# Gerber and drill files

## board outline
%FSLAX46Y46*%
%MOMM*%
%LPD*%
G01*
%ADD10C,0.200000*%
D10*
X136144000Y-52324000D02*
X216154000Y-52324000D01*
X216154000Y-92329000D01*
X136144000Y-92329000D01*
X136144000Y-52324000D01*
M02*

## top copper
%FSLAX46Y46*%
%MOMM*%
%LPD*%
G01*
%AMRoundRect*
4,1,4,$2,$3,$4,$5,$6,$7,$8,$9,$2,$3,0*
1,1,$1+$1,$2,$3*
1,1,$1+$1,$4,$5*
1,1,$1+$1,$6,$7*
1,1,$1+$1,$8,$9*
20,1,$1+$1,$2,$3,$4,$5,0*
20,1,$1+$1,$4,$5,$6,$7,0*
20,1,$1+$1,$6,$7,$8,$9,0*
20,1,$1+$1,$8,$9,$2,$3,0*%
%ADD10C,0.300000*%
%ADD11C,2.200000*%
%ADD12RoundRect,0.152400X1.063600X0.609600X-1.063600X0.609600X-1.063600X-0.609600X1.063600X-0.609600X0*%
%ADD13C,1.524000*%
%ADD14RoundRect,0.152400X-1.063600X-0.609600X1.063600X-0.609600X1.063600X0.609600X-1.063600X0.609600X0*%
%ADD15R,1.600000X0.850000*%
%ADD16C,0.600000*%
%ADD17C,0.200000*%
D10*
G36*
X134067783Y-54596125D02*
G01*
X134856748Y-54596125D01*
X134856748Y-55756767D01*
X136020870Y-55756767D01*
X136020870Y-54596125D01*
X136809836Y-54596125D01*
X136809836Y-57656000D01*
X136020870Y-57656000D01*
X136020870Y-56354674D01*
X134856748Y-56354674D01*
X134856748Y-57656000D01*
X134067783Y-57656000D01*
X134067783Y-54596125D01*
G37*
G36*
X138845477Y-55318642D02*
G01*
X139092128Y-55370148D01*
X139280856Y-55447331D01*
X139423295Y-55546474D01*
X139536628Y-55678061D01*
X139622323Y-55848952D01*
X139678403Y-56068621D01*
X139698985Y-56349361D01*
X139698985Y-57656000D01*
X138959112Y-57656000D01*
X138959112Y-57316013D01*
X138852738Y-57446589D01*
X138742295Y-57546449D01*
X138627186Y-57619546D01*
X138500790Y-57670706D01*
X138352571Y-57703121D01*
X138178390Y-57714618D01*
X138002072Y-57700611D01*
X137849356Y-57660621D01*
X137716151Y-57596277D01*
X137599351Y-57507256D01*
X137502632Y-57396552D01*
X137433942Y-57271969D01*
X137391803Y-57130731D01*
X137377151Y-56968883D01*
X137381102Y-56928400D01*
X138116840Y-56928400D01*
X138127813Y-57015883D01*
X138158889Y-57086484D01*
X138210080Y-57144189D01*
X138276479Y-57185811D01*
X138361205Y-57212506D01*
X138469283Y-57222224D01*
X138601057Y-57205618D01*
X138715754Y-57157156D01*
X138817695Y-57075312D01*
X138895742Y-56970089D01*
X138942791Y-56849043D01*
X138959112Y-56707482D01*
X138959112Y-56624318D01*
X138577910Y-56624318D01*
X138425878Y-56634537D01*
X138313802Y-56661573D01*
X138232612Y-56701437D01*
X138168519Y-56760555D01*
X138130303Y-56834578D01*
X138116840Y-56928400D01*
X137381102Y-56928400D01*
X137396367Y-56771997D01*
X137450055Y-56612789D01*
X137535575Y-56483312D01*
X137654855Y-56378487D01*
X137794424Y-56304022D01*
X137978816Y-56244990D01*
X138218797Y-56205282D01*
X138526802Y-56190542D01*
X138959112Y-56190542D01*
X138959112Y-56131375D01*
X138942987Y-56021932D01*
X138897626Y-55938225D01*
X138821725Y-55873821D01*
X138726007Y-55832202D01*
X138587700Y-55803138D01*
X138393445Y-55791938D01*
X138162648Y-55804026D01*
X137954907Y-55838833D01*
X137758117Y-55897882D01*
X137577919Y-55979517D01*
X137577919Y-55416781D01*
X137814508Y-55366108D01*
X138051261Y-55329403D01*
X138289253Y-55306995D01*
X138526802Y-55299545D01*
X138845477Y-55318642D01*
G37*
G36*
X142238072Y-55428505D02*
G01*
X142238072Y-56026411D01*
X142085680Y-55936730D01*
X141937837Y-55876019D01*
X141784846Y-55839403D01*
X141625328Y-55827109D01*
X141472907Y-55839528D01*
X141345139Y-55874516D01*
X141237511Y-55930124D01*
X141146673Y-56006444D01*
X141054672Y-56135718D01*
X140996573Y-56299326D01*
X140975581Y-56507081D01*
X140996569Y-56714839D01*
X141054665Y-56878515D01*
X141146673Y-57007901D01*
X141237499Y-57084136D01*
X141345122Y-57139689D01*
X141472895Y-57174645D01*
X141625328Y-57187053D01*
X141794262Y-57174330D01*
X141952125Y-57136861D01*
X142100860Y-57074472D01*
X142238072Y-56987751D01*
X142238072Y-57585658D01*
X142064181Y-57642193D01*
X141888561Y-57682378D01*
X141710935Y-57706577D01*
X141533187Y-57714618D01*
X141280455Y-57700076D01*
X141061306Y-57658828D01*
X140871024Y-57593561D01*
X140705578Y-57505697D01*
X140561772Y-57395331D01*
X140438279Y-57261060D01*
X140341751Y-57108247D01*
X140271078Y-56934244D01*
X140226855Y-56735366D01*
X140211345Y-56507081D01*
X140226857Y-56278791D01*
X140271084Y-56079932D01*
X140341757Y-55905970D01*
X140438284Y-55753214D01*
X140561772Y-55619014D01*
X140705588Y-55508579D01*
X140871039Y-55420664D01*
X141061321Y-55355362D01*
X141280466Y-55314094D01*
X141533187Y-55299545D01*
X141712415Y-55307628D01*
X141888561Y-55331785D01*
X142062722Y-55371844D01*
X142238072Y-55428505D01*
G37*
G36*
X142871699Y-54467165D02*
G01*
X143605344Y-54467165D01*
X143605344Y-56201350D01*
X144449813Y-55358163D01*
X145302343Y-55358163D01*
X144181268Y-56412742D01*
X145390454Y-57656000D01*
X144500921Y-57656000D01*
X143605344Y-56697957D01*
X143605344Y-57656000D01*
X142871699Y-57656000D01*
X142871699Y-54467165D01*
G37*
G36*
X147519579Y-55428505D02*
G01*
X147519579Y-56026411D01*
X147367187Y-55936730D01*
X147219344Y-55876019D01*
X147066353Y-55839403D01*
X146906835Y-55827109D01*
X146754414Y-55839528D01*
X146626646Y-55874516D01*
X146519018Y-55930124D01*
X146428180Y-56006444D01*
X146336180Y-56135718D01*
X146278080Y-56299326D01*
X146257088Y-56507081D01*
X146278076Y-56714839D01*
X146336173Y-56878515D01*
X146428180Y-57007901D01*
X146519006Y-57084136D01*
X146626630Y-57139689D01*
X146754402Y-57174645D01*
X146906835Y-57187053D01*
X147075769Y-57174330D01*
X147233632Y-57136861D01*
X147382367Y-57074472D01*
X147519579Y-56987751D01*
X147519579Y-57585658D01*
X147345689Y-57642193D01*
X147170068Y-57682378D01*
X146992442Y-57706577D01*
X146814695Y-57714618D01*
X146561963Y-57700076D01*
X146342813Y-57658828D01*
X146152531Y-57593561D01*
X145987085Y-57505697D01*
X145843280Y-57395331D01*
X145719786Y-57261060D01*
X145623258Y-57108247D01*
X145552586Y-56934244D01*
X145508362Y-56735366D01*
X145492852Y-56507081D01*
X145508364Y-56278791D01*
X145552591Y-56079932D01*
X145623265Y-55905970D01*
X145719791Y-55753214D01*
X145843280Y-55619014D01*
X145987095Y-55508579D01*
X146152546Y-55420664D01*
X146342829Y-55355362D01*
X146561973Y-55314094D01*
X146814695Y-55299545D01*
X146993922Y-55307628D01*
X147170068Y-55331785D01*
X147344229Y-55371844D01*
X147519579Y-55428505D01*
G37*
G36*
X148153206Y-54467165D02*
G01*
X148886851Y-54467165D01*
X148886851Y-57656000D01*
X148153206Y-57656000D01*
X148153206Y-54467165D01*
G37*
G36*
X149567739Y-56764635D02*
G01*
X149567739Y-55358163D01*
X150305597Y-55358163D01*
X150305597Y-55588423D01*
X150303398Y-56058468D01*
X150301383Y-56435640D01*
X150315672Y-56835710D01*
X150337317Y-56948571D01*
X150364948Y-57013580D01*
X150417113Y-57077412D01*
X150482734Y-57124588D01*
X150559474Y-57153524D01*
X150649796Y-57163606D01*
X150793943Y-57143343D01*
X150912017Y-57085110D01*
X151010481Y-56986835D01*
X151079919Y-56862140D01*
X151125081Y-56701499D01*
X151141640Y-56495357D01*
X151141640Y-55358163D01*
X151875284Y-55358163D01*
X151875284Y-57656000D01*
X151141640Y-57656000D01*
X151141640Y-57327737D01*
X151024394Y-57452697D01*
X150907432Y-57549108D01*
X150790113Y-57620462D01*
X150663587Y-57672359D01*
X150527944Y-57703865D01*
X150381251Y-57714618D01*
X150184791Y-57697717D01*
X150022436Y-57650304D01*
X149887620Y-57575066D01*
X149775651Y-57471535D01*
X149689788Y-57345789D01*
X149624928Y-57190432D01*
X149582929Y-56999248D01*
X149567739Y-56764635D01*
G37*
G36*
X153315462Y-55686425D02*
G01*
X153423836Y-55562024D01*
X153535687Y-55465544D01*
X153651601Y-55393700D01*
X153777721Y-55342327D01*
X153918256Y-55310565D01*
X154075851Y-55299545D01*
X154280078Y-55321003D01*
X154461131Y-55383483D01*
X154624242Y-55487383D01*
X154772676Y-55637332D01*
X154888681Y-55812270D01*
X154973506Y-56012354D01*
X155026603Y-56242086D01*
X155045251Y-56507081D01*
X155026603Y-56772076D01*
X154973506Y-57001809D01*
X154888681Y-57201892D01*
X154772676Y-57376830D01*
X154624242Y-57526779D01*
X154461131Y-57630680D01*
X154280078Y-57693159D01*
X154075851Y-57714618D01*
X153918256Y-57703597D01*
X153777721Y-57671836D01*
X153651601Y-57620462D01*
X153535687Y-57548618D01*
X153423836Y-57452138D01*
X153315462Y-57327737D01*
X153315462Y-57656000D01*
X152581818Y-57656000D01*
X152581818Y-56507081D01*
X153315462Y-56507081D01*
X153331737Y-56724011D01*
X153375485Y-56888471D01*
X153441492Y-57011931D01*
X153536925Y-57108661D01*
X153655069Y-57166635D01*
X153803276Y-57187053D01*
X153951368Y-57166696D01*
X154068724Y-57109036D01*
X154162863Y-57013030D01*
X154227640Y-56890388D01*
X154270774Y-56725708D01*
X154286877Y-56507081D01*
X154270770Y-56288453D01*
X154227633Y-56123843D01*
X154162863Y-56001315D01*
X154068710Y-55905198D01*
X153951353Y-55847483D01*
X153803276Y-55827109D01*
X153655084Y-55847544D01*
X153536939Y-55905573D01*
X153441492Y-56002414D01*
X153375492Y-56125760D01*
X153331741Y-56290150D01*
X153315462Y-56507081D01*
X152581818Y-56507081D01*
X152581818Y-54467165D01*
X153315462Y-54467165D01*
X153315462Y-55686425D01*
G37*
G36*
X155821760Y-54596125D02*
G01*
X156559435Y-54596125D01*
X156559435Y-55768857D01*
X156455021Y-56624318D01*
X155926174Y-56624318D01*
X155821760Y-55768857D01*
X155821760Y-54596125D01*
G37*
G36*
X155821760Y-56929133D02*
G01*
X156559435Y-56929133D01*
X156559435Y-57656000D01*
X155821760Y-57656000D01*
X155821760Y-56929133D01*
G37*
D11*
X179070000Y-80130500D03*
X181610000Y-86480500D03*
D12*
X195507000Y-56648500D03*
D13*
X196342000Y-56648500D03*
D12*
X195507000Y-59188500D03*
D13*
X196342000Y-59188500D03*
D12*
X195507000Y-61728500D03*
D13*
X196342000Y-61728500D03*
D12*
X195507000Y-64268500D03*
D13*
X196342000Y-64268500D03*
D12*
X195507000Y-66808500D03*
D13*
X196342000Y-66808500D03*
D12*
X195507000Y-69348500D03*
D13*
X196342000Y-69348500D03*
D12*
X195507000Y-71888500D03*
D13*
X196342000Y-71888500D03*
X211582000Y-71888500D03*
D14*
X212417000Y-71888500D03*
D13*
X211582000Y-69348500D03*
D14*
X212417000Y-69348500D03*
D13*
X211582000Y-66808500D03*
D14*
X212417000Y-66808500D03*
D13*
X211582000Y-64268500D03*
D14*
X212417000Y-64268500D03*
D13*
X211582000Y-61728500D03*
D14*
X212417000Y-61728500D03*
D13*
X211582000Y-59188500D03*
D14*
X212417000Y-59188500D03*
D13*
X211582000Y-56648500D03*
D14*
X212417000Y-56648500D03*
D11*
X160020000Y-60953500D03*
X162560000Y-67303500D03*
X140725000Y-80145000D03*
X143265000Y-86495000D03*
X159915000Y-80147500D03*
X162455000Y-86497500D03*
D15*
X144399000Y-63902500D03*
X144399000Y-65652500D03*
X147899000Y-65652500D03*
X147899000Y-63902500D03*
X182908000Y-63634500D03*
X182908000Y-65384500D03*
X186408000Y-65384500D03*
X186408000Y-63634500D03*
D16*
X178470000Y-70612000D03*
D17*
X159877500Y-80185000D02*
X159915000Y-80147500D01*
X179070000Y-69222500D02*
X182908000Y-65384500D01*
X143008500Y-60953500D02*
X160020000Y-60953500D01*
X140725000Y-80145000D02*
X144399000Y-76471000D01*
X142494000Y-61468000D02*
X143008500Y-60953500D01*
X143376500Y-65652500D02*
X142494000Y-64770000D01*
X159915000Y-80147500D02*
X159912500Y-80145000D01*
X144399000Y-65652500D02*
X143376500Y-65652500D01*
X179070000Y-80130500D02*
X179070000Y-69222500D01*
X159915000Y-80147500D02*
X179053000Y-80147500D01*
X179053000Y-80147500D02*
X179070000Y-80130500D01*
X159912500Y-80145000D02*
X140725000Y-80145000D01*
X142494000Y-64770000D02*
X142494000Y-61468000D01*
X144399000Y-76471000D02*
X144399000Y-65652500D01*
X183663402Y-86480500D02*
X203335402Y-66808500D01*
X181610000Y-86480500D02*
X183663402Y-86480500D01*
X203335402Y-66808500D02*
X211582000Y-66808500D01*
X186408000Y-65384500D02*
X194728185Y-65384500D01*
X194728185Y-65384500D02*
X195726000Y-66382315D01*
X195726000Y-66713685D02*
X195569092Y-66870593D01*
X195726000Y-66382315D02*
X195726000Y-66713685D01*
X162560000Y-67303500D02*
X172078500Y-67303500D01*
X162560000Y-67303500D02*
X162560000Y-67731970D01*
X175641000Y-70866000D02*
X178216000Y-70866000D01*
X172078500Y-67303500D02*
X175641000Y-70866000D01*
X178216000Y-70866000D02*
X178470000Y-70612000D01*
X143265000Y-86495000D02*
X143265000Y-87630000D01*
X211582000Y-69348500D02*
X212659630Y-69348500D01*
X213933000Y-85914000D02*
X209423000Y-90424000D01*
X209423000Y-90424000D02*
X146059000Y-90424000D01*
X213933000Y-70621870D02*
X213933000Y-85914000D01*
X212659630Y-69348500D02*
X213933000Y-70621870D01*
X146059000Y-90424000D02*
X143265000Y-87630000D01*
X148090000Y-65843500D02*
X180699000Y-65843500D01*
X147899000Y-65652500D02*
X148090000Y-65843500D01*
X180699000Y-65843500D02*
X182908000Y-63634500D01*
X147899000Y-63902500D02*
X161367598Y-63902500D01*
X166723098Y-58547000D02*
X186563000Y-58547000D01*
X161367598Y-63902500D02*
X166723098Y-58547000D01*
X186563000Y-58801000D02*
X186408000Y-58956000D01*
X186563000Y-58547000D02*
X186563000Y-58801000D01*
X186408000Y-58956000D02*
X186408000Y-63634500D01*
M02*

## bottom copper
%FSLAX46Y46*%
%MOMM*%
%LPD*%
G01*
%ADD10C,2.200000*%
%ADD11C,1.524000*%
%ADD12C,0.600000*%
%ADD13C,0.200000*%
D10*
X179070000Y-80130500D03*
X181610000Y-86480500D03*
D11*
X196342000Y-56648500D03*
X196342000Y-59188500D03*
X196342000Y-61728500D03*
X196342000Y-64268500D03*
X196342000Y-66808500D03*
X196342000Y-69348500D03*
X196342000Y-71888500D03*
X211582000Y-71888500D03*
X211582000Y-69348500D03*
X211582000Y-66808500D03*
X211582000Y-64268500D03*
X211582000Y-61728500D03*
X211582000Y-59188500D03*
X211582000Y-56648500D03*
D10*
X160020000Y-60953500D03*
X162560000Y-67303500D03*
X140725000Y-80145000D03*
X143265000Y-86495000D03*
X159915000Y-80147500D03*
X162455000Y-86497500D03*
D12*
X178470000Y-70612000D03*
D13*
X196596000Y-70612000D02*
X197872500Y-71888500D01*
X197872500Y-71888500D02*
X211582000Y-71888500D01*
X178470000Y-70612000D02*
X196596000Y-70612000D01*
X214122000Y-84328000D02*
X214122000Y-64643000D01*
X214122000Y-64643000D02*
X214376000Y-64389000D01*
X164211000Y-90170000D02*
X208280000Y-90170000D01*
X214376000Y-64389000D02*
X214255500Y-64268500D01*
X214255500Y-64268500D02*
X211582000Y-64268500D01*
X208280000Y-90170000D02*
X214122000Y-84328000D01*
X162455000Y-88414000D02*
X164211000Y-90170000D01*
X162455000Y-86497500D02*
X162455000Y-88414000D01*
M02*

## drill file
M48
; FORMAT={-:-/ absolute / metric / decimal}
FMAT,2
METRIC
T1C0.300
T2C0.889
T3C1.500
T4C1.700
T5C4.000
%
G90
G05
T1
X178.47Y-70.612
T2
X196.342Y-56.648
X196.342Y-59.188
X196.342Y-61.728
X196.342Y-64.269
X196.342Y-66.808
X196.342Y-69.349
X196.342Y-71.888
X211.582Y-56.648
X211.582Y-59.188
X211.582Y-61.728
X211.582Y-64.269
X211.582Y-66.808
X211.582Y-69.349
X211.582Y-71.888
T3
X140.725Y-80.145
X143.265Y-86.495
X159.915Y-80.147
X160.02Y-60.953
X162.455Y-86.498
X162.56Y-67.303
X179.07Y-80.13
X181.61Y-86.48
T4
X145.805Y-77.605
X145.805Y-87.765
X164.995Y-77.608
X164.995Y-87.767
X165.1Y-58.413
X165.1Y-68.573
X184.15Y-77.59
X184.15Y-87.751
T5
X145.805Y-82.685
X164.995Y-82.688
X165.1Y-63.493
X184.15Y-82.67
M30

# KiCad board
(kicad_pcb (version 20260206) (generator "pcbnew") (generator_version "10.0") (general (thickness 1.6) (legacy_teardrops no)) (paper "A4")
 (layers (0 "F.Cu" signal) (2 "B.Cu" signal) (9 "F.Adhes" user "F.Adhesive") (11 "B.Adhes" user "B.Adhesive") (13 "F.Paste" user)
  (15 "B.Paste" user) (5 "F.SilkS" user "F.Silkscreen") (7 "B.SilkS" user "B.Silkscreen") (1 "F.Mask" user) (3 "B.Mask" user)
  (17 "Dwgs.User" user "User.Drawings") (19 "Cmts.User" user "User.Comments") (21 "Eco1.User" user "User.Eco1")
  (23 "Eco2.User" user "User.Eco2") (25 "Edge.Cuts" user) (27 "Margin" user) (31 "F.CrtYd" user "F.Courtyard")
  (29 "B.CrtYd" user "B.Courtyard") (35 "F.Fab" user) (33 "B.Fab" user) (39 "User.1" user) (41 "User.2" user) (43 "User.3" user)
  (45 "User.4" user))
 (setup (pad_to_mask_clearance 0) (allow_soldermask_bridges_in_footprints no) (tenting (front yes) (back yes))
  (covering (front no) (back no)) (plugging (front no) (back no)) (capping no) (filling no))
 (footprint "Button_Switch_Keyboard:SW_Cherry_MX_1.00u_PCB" (layer "F.Cu") (at 179.07 80.1305 90)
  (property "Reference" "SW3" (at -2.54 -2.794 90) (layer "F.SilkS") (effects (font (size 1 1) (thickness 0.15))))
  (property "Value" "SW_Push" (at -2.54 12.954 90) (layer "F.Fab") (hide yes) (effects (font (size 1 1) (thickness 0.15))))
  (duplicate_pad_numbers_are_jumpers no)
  (pad "" np_thru_hole circle (at -7.62 5.08 90) (size 1.7 1.7) (drill 1.7) (layers "*.Cu" "*.Mask"))
  (pad "" np_thru_hole circle (at -2.54 5.08 90) (size 4 4) (drill 4) (layers "*.Cu" "*.Mask"))
  (pad "" np_thru_hole circle (at 2.54 5.08 90) (size 1.7 1.7) (drill 1.7) (layers "*.Cu" "*.Mask"))
  (pad "1" thru_hole circle (at 0 0 90) (size 2.2 2.2) (drill 1.5) (layers "*.Cu" "*.Mask") (remove_unused_layers no) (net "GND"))
  (pad "2" thru_hole circle (at -6.35 2.54 90) (size 2.2 2.2) (drill 1.5) (layers "*.Cu" "*.Mask") (remove_unused_layers no)
   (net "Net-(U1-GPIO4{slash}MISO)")))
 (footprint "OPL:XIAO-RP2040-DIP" (layer "F.Cu") (at 203.962 64.2685)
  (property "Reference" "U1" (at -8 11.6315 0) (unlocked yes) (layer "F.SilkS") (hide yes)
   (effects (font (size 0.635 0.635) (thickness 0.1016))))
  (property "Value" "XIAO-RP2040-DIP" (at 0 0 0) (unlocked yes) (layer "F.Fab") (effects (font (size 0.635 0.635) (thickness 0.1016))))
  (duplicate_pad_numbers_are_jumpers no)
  (pad "1" smd roundrect (at -8.455 -7.62 180) (size 2.432 1.524) (layers "F.Cu" "F.Mask") (roundrect_rratio 0.1)
   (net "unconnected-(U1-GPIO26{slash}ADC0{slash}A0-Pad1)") (thermal_bridge_angle 45))
  (pad "1" thru_hole circle (at -7.62 -7.62 180) (size 1.524 1.524) (drill 0.889) (layers "*.Cu" "*.Mask") (remove_unused_layers no)
   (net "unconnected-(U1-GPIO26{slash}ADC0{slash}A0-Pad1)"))
  (pad "2" smd roundrect (at -8.455 -5.08 180) (size 2.432 1.524) (layers "F.Cu" "F.Mask") (roundrect_rratio 0.1)
   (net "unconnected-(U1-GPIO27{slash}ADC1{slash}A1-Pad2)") (thermal_bridge_angle 45))
  (pad "2" thru_hole circle (at -7.62 -5.08 180) (size 1.524 1.524) (drill 0.889) (layers "*.Cu" "*.Mask") (remove_unused_layers no)
   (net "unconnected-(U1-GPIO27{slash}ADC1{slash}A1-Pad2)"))
  (pad "3" smd roundrect (at -8.455 -2.54 180) (size 2.432 1.524) (layers "F.Cu" "F.Mask") (roundrect_rratio 0.1)
   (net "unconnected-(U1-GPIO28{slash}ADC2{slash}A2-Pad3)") (thermal_bridge_angle 45))
  (pad "3" thru_hole circle (at -7.62 -2.54 180) (size 1.524 1.524) (drill 0.889) (layers "*.Cu" "*.Mask") (remove_unused_layers no)
   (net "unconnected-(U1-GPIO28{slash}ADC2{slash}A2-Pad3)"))
  (pad "4" smd roundrect (at -8.455 0 180) (size 2.432 1.524) (layers "F.Cu" "F.Mask") (roundrect_rratio 0.1)
   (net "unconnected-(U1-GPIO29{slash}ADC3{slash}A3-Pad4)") (thermal_bridge_angle 45))
  (pad "4" thru_hole circle (at -7.62 0 180) (size 1.524 1.524) (drill 0.889) (layers "*.Cu" "*.Mask") (remove_unused_layers no)
   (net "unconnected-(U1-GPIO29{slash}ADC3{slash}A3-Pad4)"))
  (pad "5" smd roundrect (at -8.455 2.54 180) (size 2.432 1.524) (layers "F.Cu" "F.Mask") (roundrect_rratio 0.1) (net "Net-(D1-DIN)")
   (thermal_bridge_angle 45))
  (pad "5" thru_hole circle (at -7.62 2.54 180) (size 1.524 1.524) (drill 0.889) (layers "*.Cu" "*.Mask") (remove_unused_layers no)
   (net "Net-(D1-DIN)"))
  (pad "6" smd roundrect (at -8.455 5.08 180) (size 2.432 1.524) (layers "F.Cu" "F.Mask") (roundrect_rratio 0.1)
   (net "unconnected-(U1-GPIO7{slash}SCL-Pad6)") (thermal_bridge_angle 45))
  (pad "6" thru_hole circle (at -7.62 5.08 180) (size 1.524 1.524) (drill 0.889) (layers "*.Cu" "*.Mask") (remove_unused_layers no)
   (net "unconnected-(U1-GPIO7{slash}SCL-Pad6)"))
  (pad "7" smd roundrect (at -8.455 7.62 180) (size 2.432 1.524) (layers "F.Cu" "F.Mask") (roundrect_rratio 0.1)
   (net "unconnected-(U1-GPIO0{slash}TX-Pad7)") (thermal_bridge_angle 45))
  (pad "7" thru_hole circle (at -7.62 7.62 180) (size 1.524 1.524) (drill 0.889) (layers "*.Cu" "*.Mask") (remove_unused_layers no)
   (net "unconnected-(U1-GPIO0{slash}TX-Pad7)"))
  (pad "8" thru_hole circle (at 7.62 7.62) (size 1.524 1.524) (drill 0.889) (layers "*.Cu" "*.Mask") (remove_unused_layers no)
   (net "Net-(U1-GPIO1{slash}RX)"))
  (pad "8" smd roundrect (at 8.455 7.62) (size 2.432 1.524) (layers "F.Cu" "F.Mask") (roundrect_rratio 0.1) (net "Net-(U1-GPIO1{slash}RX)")
   (thermal_bridge_angle 45))
  (pad "9" thru_hole circle (at 7.62 5.08) (size 1.524 1.524) (drill 0.889) (layers "*.Cu" "*.Mask") (remove_unused_layers no)
   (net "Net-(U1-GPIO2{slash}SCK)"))
  (pad "9" smd roundrect (at 8.455 5.08) (size 2.432 1.524) (layers "F.Cu" "F.Mask") (roundrect_rratio 0.1) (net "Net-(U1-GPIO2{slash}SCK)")
   (thermal_bridge_angle 45))
  (pad "10" thru_hole circle (at 7.62 2.54) (size 1.524 1.524) (drill 0.889) (layers "*.Cu" "*.Mask") (remove_unused_layers no)
   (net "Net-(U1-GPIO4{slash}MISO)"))
  (pad "10" smd roundrect (at 8.455 2.54) (size 2.432 1.524) (layers "F.Cu" "F.Mask") (roundrect_rratio 0.1)
   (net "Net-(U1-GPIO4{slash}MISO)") (thermal_bridge_angle 45))
  (pad "11" thru_hole circle (at 7.62 0) (size 1.524 1.524) (drill 0.889) (layers "*.Cu" "*.Mask") (remove_unused_layers no)
   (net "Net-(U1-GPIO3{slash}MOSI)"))
  (pad "11" smd roundrect (at 8.455 0) (size 2.432 1.524) (layers "F.Cu" "F.Mask") (roundrect_rratio 0.1) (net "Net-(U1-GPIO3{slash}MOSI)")
   (thermal_bridge_angle 45))
  (pad "12" thru_hole circle (at 7.62 -2.54) (size 1.524 1.524) (drill 0.889) (layers "*.Cu" "*.Mask") (remove_unused_layers no)
   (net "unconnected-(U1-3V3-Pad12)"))
  (pad "12" smd roundrect (at 8.455 -2.54) (size 2.432 1.524) (layers "F.Cu" "F.Mask") (roundrect_rratio 0.1)
   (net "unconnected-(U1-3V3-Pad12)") (thermal_bridge_angle 45))
  (pad "13" thru_hole circle (at 7.62 -5.08) (size 1.524 1.524) (drill 0.889) (layers "*.Cu" "*.Mask") (remove_unused_layers no)
   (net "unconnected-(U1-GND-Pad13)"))
  (pad "13" smd roundrect (at 8.455 -5.08) (size 2.432 1.524) (layers "F.Cu" "F.Mask") (roundrect_rratio 0.1)
   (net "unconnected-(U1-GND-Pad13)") (thermal_bridge_angle 45))
  (pad "14" thru_hole circle (at 7.62 -7.62) (size 1.524 1.524) (drill 0.889) (layers "*.Cu" "*.Mask") (remove_unused_layers no)
   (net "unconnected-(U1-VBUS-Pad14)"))
  (pad "14" smd roundrect (at 8.455 -7.62) (size 2.432 1.524) (layers "F.Cu" "F.Mask") (roundrect_rratio 0.1)
   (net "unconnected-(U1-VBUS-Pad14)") (thermal_bridge_angle 45)))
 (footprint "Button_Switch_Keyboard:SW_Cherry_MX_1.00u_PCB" (layer "F.Cu") (at 160.02 60.9535 90)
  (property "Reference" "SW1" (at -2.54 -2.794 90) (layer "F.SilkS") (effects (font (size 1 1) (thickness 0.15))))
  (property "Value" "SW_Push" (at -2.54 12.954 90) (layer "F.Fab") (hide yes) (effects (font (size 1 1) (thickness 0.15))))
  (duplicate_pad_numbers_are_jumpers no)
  (pad "" np_thru_hole circle (at -7.62 5.08 90) (size 1.7 1.7) (drill 1.7) (layers "*.Cu" "*.Mask"))
  (pad "" np_thru_hole circle (at -2.54 5.08 90) (size 4 4) (drill 4) (layers "*.Cu" "*.Mask"))
  (pad "" np_thru_hole circle (at 2.54 5.08 90) (size 1.7 1.7) (drill 1.7) (layers "*.Cu" "*.Mask"))
  (pad "1" thru_hole circle (at 0 0 90) (size 2.2 2.2) (drill 1.5) (layers "*.Cu" "*.Mask") (remove_unused_layers no) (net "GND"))
  (pad "2" thru_hole circle (at -6.35 2.54 90) (size 2.2 2.2) (drill 1.5) (layers "*.Cu" "*.Mask") (remove_unused_layers no)
   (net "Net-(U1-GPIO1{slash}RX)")))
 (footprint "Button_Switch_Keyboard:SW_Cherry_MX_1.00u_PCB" (layer "F.Cu") (at 140.725 80.145 90)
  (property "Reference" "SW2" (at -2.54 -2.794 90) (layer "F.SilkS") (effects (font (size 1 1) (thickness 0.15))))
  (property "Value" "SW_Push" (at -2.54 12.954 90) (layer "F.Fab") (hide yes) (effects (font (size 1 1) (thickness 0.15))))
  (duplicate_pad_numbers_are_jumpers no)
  (pad "" np_thru_hole circle (at -7.62 5.08 90) (size 1.7 1.7) (drill 1.7) (layers "*.Cu" "*.Mask"))
  (pad "" np_thru_hole circle (at -2.54 5.08 90) (size 4 4) (drill 4) (layers "*.Cu" "*.Mask"))
  (pad "" np_thru_hole circle (at 2.54 5.08 90) (size 1.7 1.7) (drill 1.7) (layers "*.Cu" "*.Mask"))
  (pad "1" thru_hole circle (at 0 0 90) (size 2.2 2.2) (drill 1.5) (layers "*.Cu" "*.Mask") (remove_unused_layers no) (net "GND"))
  (pad "2" thru_hole circle (at -6.35 2.54 90) (size 2.2 2.2) (drill 1.5) (layers "*.Cu" "*.Mask") (remove_unused_layers no)
   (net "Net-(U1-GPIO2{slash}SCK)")))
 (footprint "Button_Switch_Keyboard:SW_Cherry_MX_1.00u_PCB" (layer "F.Cu") (at 159.915 80.1475 90)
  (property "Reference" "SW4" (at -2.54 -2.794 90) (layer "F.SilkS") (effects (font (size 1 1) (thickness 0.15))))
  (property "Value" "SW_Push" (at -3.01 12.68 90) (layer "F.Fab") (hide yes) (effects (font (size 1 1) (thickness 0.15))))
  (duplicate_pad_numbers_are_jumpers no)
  (pad "" np_thru_hole circle (at -7.62 5.08 90) (size 1.7 1.7) (drill 1.7) (layers "*.Cu" "*.Mask"))
  (pad "" np_thru_hole circle (at -2.54 5.08 90) (size 4 4) (drill 4) (layers "*.Cu" "*.Mask"))
  (pad "" np_thru_hole circle (at 2.54 5.08 90) (size 1.7 1.7) (drill 1.7) (layers "*.Cu" "*.Mask"))
  (pad "1" thru_hole circle (at 0 0 90) (size 2.2 2.2) (drill 1.5) (layers "*.Cu" "*.Mask") (remove_unused_layers no) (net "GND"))
  (pad "2" thru_hole circle (at -6.35 2.54 90) (size 2.2 2.2) (drill 1.5) (layers "*.Cu" "*.Mask") (remove_unused_layers no)
   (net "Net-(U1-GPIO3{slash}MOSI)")))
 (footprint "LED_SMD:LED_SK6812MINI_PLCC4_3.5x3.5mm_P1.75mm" (layer "F.Cu") (at 146.149 64.7775)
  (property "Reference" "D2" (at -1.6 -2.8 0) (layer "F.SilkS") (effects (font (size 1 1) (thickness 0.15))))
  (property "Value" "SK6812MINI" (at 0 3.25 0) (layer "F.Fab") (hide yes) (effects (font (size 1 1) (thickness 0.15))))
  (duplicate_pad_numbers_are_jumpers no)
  (pad "1" smd rect (at -1.75 -0.875) (size 1.6 0.85) (layers "F.Cu" "F.Mask" "F.Paste") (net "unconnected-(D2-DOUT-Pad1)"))
  (pad "2" smd rect (at -1.75 0.875) (size 1.6 0.85) (layers "F.Cu" "F.Mask" "F.Paste") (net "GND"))
  (pad "3" smd rect (at 1.75 0.875) (size 1.6 0.85) (layers "F.Cu" "F.Mask" "F.Paste") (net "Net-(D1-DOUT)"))
  (pad "4" smd rect (at 1.75 -0.875) (size 1.6 0.85) (layers "F.Cu" "F.Mask" "F.Paste") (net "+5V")))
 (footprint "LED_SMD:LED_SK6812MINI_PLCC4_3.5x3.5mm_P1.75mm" (layer "F.Cu") (at 184.658 64.5095)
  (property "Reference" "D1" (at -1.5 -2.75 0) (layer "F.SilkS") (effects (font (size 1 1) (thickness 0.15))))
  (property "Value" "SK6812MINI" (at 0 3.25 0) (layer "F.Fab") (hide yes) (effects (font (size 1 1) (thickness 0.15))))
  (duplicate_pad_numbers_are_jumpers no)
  (pad "1" smd rect (at -1.75 -0.875) (size 1.6 0.85) (layers "F.Cu" "F.Mask" "F.Paste") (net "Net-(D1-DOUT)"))
  (pad "2" smd rect (at -1.75 0.875) (size 1.6 0.85) (layers "F.Cu" "F.Mask" "F.Paste") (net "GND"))
  (pad "3" smd rect (at 1.75 0.875) (size 1.6 0.85) (layers "F.Cu" "F.Mask" "F.Paste") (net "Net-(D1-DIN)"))
  (pad "4" smd rect (at 1.75 -0.875) (size 1.6 0.85) (layers "F.Cu" "F.Mask" "F.Paste") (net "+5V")))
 (gr_rect (start 136.144 52.324) (end 216.154 92.329) (stroke (width 0.2) (type default)) (fill no) (layer "Edge.Cuts"))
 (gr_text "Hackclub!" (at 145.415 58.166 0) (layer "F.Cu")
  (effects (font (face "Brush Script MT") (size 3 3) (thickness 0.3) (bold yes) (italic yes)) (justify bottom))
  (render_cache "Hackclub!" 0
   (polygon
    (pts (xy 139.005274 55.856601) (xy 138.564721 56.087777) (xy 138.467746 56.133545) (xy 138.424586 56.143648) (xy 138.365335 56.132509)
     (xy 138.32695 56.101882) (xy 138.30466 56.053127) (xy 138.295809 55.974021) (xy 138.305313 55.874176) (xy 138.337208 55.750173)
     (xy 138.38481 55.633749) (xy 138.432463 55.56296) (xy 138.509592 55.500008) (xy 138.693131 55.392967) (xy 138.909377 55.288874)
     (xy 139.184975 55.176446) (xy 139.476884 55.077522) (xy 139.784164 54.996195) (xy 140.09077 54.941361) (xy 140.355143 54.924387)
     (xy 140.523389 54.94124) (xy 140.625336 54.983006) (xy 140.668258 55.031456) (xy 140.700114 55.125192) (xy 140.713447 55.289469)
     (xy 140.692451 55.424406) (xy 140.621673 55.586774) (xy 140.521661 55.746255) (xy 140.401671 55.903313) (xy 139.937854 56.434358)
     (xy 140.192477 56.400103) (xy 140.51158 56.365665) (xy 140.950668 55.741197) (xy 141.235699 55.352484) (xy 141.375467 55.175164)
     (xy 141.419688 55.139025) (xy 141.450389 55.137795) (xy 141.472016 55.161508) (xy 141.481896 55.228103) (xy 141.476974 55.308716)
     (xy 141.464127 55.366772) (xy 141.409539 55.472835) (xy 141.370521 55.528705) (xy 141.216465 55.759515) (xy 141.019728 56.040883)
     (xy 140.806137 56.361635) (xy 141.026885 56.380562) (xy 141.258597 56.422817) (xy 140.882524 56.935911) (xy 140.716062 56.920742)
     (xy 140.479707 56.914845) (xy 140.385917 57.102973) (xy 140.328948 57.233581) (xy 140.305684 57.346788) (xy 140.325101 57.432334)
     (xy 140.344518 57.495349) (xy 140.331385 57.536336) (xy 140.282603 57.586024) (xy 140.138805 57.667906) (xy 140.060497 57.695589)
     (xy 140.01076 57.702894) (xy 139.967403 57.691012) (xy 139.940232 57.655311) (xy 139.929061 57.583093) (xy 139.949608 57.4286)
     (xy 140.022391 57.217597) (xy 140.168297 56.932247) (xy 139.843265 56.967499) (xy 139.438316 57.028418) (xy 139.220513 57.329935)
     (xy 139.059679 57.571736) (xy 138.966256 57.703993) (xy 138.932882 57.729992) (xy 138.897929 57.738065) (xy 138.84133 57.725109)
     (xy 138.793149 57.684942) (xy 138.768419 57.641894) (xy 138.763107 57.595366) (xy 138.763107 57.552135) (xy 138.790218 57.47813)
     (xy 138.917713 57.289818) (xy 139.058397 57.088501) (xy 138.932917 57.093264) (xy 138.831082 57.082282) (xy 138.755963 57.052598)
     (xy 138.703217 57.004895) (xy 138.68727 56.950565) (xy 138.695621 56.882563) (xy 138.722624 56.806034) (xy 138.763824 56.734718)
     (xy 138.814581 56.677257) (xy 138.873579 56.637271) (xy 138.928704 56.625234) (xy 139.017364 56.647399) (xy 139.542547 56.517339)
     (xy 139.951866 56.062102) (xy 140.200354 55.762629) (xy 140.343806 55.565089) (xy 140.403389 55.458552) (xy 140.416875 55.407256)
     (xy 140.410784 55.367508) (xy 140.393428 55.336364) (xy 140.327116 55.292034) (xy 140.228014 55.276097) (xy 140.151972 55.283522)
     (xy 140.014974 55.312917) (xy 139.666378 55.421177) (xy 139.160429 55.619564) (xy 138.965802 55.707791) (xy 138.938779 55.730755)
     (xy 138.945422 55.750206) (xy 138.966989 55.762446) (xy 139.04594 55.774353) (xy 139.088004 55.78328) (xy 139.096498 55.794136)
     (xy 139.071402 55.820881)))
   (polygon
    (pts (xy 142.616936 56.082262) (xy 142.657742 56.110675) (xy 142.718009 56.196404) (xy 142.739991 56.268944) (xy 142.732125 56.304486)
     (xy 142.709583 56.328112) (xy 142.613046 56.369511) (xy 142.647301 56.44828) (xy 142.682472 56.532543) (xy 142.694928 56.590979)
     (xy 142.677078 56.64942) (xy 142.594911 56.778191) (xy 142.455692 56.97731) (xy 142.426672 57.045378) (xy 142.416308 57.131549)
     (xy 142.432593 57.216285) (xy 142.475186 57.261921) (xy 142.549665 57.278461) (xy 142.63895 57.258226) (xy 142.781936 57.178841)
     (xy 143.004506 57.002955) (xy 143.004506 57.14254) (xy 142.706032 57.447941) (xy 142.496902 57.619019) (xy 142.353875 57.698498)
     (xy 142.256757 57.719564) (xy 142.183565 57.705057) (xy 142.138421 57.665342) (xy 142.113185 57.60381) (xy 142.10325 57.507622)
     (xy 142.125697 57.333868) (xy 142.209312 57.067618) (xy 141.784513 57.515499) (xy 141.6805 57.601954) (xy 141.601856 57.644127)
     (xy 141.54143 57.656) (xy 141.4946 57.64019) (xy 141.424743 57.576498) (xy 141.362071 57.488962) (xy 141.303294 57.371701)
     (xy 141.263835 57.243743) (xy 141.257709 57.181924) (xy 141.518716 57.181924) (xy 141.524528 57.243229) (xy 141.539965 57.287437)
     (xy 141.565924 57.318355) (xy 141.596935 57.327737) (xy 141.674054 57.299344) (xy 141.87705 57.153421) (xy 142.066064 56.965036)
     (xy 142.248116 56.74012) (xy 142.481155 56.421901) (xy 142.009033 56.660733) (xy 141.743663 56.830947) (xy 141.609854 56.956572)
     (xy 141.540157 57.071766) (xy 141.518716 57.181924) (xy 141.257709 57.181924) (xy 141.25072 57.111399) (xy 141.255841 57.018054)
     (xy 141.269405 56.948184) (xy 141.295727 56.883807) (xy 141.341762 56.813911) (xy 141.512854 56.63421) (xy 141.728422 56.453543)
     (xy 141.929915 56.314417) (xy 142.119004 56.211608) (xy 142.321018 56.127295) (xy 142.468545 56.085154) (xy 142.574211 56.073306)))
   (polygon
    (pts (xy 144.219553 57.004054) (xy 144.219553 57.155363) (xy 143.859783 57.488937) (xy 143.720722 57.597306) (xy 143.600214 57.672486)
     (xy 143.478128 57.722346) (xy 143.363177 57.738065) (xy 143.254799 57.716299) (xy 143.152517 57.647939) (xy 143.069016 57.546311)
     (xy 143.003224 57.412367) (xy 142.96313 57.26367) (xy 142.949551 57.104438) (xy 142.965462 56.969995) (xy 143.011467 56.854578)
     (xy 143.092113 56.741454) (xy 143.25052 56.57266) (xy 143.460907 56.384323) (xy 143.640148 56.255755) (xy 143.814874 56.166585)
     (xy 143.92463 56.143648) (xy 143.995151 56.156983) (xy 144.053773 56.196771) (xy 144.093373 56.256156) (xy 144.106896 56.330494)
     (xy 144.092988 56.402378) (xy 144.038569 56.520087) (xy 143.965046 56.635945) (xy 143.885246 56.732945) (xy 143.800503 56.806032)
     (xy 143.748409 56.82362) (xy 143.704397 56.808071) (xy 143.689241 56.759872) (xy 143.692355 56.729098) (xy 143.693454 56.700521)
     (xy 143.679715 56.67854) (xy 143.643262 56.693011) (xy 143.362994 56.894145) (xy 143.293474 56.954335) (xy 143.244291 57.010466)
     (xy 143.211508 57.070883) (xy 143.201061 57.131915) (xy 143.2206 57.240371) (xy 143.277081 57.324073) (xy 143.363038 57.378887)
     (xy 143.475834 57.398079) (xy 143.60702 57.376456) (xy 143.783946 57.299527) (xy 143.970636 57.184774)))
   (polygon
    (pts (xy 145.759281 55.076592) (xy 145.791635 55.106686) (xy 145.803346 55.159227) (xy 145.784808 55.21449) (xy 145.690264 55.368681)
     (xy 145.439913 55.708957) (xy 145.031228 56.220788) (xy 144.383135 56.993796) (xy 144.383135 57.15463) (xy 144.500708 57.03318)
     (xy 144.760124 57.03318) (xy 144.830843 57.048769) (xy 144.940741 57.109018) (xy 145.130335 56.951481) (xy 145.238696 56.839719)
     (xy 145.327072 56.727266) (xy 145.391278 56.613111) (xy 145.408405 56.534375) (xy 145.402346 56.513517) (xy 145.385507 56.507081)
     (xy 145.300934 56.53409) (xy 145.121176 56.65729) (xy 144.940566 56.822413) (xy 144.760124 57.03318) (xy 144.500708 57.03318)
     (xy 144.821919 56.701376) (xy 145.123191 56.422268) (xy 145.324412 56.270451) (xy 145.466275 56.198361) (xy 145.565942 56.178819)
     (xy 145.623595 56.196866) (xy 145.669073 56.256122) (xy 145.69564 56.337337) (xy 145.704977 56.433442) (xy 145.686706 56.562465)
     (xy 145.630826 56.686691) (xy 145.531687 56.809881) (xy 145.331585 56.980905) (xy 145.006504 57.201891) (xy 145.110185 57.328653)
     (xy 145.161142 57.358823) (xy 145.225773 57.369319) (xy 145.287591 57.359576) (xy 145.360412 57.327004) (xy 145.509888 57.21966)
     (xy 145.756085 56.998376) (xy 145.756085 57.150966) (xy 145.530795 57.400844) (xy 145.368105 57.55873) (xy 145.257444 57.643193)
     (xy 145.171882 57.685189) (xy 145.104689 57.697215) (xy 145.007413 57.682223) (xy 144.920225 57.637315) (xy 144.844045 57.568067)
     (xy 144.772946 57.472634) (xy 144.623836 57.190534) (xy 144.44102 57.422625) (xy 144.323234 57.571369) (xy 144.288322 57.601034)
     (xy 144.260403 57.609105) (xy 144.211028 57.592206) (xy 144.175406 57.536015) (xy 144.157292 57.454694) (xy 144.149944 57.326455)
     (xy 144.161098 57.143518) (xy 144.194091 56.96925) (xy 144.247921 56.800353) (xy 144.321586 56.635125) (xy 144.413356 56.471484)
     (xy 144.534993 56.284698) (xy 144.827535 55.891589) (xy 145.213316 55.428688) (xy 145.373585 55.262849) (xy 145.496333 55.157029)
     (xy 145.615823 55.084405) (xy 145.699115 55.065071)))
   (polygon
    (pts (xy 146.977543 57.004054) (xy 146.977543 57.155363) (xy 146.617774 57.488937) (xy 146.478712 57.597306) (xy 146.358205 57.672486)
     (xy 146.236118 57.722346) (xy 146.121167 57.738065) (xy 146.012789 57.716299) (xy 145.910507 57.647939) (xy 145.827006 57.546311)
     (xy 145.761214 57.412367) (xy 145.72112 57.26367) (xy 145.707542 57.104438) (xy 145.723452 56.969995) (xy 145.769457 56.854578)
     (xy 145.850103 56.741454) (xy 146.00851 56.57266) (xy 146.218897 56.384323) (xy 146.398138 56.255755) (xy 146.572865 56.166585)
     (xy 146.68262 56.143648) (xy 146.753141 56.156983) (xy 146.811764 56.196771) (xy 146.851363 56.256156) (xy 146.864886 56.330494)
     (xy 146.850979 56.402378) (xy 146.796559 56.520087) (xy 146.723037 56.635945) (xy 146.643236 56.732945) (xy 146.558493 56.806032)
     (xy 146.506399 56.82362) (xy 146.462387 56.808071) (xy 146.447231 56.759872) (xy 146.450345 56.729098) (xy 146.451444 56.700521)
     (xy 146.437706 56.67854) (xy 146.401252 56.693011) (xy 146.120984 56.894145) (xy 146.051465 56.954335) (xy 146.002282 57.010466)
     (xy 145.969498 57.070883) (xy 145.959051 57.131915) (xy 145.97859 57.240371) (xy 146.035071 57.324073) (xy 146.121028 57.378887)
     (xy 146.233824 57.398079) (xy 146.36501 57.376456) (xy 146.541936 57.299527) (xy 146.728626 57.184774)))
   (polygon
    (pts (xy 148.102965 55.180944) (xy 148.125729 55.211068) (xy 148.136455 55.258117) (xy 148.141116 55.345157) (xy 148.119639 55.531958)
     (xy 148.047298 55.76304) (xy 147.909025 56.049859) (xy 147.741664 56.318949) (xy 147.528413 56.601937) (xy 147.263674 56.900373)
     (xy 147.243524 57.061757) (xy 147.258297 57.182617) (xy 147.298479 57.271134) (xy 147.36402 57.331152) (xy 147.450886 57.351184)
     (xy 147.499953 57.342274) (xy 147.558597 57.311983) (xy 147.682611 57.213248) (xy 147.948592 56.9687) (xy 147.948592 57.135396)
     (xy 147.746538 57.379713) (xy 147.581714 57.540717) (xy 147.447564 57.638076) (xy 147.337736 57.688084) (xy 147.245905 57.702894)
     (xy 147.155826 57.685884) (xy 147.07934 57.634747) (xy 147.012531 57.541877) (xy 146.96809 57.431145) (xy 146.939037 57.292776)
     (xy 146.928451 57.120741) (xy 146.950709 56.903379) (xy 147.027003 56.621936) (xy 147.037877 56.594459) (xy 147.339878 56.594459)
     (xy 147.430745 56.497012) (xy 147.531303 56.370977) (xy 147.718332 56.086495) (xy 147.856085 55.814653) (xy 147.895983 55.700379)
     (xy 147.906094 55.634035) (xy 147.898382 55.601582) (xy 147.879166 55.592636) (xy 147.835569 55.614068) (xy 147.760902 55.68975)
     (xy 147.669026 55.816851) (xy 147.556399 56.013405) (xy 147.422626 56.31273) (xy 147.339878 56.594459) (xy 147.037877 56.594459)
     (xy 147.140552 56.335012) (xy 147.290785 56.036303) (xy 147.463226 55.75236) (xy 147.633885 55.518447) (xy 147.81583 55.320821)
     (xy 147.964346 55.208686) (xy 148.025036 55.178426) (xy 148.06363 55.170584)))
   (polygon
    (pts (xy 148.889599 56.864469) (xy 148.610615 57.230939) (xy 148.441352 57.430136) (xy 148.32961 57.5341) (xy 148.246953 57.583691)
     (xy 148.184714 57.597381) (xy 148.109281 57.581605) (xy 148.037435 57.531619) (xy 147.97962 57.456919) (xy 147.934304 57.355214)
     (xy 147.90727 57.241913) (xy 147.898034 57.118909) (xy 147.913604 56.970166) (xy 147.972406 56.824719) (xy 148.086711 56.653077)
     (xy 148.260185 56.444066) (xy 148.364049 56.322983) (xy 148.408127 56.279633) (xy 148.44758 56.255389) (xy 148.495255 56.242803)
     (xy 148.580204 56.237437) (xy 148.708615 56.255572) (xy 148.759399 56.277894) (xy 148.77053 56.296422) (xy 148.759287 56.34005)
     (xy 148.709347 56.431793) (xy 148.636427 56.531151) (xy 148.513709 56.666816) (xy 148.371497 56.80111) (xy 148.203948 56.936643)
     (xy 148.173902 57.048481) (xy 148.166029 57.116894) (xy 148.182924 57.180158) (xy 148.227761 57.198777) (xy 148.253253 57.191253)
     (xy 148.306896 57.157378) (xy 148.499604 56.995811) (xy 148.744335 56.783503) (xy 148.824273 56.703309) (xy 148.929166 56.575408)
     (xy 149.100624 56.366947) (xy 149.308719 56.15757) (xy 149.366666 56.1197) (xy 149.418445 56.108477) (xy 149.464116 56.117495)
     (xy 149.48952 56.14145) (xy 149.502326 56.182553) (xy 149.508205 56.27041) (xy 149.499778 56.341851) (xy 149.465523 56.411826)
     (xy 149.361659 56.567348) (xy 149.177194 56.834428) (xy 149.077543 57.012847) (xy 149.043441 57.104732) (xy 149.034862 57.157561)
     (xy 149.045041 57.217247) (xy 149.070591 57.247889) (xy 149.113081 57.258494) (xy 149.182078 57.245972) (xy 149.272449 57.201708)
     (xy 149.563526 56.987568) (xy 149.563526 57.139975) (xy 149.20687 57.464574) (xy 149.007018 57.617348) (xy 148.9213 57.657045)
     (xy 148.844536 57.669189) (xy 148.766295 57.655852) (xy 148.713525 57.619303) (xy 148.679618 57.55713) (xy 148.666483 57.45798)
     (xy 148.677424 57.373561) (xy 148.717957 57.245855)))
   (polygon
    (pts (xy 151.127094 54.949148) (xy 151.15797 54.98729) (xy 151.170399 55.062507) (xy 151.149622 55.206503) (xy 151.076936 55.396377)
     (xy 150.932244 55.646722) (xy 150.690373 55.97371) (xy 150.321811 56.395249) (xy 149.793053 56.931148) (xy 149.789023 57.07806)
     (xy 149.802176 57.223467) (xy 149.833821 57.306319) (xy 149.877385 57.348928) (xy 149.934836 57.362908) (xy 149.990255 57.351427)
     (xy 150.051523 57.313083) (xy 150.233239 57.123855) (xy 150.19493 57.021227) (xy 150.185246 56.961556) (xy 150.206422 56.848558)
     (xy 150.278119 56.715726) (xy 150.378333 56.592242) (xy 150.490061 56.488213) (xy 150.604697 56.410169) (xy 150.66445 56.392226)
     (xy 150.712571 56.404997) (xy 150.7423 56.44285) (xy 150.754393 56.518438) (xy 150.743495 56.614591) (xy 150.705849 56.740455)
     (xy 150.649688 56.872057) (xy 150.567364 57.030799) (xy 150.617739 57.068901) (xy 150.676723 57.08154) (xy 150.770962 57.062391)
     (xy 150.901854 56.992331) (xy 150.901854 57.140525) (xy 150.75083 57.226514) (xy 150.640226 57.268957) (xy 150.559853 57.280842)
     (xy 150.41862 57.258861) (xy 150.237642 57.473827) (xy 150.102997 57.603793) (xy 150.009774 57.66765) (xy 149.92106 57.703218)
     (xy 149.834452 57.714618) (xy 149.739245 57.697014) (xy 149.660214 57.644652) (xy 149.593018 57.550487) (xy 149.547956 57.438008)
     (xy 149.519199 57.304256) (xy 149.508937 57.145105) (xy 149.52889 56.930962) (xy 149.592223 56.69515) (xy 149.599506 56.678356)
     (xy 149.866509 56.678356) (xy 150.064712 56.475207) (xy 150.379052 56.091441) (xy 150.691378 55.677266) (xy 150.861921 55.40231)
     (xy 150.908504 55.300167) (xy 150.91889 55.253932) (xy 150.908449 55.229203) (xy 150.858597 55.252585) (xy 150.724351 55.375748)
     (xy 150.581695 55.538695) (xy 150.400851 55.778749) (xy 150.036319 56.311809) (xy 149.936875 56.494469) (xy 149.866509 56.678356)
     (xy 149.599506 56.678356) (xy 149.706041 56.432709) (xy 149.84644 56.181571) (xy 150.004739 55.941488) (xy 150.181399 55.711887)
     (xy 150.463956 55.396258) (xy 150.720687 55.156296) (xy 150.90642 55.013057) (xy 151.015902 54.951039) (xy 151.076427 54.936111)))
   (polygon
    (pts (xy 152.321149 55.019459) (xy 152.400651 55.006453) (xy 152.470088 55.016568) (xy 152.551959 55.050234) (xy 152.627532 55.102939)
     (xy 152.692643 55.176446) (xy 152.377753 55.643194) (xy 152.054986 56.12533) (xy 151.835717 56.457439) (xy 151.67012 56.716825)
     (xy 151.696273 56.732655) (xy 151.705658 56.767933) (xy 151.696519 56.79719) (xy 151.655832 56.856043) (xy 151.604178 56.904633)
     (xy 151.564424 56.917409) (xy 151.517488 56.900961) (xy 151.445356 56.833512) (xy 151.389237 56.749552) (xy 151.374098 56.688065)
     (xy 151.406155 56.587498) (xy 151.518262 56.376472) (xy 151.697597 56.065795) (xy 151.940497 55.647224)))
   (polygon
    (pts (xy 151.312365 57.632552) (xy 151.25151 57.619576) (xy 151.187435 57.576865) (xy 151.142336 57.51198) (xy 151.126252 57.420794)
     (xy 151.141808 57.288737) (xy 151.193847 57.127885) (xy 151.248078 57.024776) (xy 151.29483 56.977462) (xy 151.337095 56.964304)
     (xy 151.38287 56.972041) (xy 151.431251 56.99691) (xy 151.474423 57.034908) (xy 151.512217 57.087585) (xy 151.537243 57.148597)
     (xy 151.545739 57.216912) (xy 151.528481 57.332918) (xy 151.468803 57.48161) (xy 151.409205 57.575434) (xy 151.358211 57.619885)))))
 (segment (start 159.8775 80.185) (end 159.915 80.1475) (width 0.2) (layer "F.Cu") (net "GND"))
 (segment (start 179.07 69.2225) (end 182.908 65.3845) (width 0.2) (layer "F.Cu") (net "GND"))
 (segment (start 143.0085 60.9535) (end 160.02 60.9535) (width 0.2) (layer "F.Cu") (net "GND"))
 (segment (start 140.725 80.145) (end 144.399 76.471) (width 0.2) (layer "F.Cu") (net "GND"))
 (segment (start 142.494 61.468) (end 143.0085 60.9535) (width 0.2) (layer "F.Cu") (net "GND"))
 (segment (start 143.3765 65.6525) (end 142.494 64.77) (width 0.2) (layer "F.Cu") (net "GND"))
 (segment (start 159.915 80.1475) (end 159.9125 80.145) (width 0.2) (layer "F.Cu") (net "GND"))
 (segment (start 144.399 65.6525) (end 143.3765 65.6525) (width 0.2) (layer "F.Cu") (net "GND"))
 (segment (start 179.07 80.1305) (end 179.07 69.2225) (width 0.2) (layer "F.Cu") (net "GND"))
 (segment (start 159.915 80.1475) (end 179.053 80.1475) (width 0.2) (layer "F.Cu") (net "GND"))
 (segment (start 179.053 80.1475) (end 179.07 80.1305) (width 0.2) (layer "F.Cu") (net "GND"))
 (segment (start 159.9125 80.145) (end 140.725 80.145) (width 0.2) (layer "F.Cu") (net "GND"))
 (segment (start 142.494 64.77) (end 142.494 61.468) (width 0.2) (layer "F.Cu") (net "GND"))
 (segment (start 144.399 76.471) (end 144.399 65.6525) (width 0.2) (layer "F.Cu") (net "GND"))
 (segment (start 183.663402 86.4805) (end 203.335402 66.8085) (width 0.2) (layer "F.Cu") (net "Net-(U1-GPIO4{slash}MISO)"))
 (segment (start 181.61 86.4805) (end 183.663402 86.4805) (width 0.2) (layer "F.Cu") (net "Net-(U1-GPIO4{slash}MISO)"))
 (segment (start 203.335402 66.8085) (end 211.582 66.8085) (width 0.2) (layer "F.Cu") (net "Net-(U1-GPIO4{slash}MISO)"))
 (segment (start 186.408 65.3845) (end 194.728185 65.3845) (width 0.2) (layer "F.Cu") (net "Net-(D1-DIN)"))
 (segment (start 194.728185 65.3845) (end 195.726 66.382315) (width 0.2) (layer "F.Cu") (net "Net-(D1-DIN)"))
 (segment (start 195.726 66.713685) (end 195.569092 66.870593) (width 0.2) (layer "F.Cu") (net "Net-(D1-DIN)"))
 (segment (start 195.726 66.382315) (end 195.726 66.713685) (width 0.2) (layer "F.Cu") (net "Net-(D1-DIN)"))
 (segment (start 162.56 67.3035) (end 172.0785 67.3035) (width 0.2) (layer "F.Cu") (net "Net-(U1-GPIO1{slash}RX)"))
 (segment (start 162.56 67.3035) (end 162.56 67.73197) (width 0.2) (layer "F.Cu") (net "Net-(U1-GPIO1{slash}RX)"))
 (segment (start 175.641 70.866) (end 178.216 70.866) (width 0.2) (layer "F.Cu") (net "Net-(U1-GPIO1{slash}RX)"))
 (segment (start 172.0785 67.3035) (end 175.641 70.866) (width 0.2) (layer "F.Cu") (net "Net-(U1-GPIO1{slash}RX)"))
 (segment (start 178.216 70.866) (end 178.47 70.612) (width 0.2) (layer "F.Cu") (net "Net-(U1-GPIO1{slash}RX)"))
 (via (at 178.47 70.612) (size 0.6) (drill 0.3) (layers "F.Cu" "B.Cu") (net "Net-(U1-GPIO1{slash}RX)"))
 (segment (start 196.596 70.612) (end 197.8725 71.8885) (width 0.2) (layer "B.Cu") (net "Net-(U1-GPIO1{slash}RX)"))
 (segment (start 197.8725 71.8885) (end 211.582 71.8885) (width 0.2) (layer "B.Cu") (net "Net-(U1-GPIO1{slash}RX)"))
 (segment (start 178.47 70.612) (end 196.596 70.612) (width 0.2) (layer "B.Cu") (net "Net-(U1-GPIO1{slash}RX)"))
 (segment (start 143.265 86.495) (end 143.265 87.63) (width 0.2) (layer "F.Cu") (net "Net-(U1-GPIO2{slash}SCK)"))
 (segment (start 211.582 69.3485) (end 212.65963 69.3485) (width 0.2) (layer "F.Cu") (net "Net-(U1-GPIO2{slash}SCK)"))
 (segment (start 213.933 85.914) (end 209.423 90.424) (width 0.2) (layer "F.Cu") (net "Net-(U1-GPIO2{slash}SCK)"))
 (segment (start 209.423 90.424) (end 146.059 90.424) (width 0.2) (layer "F.Cu") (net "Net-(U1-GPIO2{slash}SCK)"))
 (segment (start 213.933 70.62187) (end 213.933 85.914) (width 0.2) (layer "F.Cu") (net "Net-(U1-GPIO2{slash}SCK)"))
 (segment (start 212.65963 69.3485) (end 213.933 70.62187) (width 0.2) (layer "F.Cu") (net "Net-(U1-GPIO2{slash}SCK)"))
 (segment (start 146.059 90.424) (end 143.265 87.63) (width 0.2) (layer "F.Cu") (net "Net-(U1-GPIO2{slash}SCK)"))
 (segment (start 214.122 84.328) (end 214.122 64.643) (width 0.2) (layer "B.Cu") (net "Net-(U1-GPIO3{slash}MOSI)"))
 (segment (start 214.122 64.643) (end 214.376 64.389) (width 0.2) (layer "B.Cu") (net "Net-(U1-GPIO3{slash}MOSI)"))
 (segment (start 164.211 90.17) (end 208.28 90.17) (width 0.2) (layer "B.Cu") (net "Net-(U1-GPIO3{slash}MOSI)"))
 (segment (start 214.376 64.389) (end 214.2555 64.2685) (width 0.2) (layer "B.Cu") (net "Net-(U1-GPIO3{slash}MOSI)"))
 (segment (start 214.2555 64.2685) (end 211.582 64.2685) (width 0.2) (layer "B.Cu") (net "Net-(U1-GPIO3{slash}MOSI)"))
 (segment (start 208.28 90.17) (end 214.122 84.328) (width 0.2) (layer "B.Cu") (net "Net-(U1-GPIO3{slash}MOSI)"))
 (segment (start 162.455 88.414) (end 164.211 90.17) (width 0.2) (layer "B.Cu") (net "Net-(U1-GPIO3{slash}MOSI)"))
 (segment (start 162.455 86.4975) (end 162.455 88.414) (width 0.2) (layer "B.Cu") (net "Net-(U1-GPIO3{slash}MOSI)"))
 (segment (start 148.09 65.8435) (end 180.699 65.8435) (width 0.2) (layer "F.Cu") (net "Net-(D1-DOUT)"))
 (segment (start 147.899 65.6525) (end 148.09 65.8435) (width 0.2) (layer "F.Cu") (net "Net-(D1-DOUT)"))
 (segment (start 180.699 65.8435) (end 182.908 63.6345) (width 0.2) (layer "F.Cu") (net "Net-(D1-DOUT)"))
 (segment (start 147.899 63.9025) (end 161.367598 63.9025) (width 0.2) (layer "F.Cu") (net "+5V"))
 (segment (start 166.723098 58.547) (end 186.563 58.547) (width 0.2) (layer "F.Cu") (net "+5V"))
 (segment (start 161.367598 63.9025) (end 166.723098 58.547) (width 0.2) (layer "F.Cu") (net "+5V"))
 (segment (start 186.563 58.801) (end 186.408 58.956) (width 0.2) (layer "F.Cu") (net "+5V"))
 (segment (start 186.563 58.547) (end 186.563 58.801) (width 0.2) (layer "F.Cu") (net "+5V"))
 (segment (start 186.408 58.956) (end 186.408 63.6345) (width 0.2) (layer "F.Cu") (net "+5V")))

